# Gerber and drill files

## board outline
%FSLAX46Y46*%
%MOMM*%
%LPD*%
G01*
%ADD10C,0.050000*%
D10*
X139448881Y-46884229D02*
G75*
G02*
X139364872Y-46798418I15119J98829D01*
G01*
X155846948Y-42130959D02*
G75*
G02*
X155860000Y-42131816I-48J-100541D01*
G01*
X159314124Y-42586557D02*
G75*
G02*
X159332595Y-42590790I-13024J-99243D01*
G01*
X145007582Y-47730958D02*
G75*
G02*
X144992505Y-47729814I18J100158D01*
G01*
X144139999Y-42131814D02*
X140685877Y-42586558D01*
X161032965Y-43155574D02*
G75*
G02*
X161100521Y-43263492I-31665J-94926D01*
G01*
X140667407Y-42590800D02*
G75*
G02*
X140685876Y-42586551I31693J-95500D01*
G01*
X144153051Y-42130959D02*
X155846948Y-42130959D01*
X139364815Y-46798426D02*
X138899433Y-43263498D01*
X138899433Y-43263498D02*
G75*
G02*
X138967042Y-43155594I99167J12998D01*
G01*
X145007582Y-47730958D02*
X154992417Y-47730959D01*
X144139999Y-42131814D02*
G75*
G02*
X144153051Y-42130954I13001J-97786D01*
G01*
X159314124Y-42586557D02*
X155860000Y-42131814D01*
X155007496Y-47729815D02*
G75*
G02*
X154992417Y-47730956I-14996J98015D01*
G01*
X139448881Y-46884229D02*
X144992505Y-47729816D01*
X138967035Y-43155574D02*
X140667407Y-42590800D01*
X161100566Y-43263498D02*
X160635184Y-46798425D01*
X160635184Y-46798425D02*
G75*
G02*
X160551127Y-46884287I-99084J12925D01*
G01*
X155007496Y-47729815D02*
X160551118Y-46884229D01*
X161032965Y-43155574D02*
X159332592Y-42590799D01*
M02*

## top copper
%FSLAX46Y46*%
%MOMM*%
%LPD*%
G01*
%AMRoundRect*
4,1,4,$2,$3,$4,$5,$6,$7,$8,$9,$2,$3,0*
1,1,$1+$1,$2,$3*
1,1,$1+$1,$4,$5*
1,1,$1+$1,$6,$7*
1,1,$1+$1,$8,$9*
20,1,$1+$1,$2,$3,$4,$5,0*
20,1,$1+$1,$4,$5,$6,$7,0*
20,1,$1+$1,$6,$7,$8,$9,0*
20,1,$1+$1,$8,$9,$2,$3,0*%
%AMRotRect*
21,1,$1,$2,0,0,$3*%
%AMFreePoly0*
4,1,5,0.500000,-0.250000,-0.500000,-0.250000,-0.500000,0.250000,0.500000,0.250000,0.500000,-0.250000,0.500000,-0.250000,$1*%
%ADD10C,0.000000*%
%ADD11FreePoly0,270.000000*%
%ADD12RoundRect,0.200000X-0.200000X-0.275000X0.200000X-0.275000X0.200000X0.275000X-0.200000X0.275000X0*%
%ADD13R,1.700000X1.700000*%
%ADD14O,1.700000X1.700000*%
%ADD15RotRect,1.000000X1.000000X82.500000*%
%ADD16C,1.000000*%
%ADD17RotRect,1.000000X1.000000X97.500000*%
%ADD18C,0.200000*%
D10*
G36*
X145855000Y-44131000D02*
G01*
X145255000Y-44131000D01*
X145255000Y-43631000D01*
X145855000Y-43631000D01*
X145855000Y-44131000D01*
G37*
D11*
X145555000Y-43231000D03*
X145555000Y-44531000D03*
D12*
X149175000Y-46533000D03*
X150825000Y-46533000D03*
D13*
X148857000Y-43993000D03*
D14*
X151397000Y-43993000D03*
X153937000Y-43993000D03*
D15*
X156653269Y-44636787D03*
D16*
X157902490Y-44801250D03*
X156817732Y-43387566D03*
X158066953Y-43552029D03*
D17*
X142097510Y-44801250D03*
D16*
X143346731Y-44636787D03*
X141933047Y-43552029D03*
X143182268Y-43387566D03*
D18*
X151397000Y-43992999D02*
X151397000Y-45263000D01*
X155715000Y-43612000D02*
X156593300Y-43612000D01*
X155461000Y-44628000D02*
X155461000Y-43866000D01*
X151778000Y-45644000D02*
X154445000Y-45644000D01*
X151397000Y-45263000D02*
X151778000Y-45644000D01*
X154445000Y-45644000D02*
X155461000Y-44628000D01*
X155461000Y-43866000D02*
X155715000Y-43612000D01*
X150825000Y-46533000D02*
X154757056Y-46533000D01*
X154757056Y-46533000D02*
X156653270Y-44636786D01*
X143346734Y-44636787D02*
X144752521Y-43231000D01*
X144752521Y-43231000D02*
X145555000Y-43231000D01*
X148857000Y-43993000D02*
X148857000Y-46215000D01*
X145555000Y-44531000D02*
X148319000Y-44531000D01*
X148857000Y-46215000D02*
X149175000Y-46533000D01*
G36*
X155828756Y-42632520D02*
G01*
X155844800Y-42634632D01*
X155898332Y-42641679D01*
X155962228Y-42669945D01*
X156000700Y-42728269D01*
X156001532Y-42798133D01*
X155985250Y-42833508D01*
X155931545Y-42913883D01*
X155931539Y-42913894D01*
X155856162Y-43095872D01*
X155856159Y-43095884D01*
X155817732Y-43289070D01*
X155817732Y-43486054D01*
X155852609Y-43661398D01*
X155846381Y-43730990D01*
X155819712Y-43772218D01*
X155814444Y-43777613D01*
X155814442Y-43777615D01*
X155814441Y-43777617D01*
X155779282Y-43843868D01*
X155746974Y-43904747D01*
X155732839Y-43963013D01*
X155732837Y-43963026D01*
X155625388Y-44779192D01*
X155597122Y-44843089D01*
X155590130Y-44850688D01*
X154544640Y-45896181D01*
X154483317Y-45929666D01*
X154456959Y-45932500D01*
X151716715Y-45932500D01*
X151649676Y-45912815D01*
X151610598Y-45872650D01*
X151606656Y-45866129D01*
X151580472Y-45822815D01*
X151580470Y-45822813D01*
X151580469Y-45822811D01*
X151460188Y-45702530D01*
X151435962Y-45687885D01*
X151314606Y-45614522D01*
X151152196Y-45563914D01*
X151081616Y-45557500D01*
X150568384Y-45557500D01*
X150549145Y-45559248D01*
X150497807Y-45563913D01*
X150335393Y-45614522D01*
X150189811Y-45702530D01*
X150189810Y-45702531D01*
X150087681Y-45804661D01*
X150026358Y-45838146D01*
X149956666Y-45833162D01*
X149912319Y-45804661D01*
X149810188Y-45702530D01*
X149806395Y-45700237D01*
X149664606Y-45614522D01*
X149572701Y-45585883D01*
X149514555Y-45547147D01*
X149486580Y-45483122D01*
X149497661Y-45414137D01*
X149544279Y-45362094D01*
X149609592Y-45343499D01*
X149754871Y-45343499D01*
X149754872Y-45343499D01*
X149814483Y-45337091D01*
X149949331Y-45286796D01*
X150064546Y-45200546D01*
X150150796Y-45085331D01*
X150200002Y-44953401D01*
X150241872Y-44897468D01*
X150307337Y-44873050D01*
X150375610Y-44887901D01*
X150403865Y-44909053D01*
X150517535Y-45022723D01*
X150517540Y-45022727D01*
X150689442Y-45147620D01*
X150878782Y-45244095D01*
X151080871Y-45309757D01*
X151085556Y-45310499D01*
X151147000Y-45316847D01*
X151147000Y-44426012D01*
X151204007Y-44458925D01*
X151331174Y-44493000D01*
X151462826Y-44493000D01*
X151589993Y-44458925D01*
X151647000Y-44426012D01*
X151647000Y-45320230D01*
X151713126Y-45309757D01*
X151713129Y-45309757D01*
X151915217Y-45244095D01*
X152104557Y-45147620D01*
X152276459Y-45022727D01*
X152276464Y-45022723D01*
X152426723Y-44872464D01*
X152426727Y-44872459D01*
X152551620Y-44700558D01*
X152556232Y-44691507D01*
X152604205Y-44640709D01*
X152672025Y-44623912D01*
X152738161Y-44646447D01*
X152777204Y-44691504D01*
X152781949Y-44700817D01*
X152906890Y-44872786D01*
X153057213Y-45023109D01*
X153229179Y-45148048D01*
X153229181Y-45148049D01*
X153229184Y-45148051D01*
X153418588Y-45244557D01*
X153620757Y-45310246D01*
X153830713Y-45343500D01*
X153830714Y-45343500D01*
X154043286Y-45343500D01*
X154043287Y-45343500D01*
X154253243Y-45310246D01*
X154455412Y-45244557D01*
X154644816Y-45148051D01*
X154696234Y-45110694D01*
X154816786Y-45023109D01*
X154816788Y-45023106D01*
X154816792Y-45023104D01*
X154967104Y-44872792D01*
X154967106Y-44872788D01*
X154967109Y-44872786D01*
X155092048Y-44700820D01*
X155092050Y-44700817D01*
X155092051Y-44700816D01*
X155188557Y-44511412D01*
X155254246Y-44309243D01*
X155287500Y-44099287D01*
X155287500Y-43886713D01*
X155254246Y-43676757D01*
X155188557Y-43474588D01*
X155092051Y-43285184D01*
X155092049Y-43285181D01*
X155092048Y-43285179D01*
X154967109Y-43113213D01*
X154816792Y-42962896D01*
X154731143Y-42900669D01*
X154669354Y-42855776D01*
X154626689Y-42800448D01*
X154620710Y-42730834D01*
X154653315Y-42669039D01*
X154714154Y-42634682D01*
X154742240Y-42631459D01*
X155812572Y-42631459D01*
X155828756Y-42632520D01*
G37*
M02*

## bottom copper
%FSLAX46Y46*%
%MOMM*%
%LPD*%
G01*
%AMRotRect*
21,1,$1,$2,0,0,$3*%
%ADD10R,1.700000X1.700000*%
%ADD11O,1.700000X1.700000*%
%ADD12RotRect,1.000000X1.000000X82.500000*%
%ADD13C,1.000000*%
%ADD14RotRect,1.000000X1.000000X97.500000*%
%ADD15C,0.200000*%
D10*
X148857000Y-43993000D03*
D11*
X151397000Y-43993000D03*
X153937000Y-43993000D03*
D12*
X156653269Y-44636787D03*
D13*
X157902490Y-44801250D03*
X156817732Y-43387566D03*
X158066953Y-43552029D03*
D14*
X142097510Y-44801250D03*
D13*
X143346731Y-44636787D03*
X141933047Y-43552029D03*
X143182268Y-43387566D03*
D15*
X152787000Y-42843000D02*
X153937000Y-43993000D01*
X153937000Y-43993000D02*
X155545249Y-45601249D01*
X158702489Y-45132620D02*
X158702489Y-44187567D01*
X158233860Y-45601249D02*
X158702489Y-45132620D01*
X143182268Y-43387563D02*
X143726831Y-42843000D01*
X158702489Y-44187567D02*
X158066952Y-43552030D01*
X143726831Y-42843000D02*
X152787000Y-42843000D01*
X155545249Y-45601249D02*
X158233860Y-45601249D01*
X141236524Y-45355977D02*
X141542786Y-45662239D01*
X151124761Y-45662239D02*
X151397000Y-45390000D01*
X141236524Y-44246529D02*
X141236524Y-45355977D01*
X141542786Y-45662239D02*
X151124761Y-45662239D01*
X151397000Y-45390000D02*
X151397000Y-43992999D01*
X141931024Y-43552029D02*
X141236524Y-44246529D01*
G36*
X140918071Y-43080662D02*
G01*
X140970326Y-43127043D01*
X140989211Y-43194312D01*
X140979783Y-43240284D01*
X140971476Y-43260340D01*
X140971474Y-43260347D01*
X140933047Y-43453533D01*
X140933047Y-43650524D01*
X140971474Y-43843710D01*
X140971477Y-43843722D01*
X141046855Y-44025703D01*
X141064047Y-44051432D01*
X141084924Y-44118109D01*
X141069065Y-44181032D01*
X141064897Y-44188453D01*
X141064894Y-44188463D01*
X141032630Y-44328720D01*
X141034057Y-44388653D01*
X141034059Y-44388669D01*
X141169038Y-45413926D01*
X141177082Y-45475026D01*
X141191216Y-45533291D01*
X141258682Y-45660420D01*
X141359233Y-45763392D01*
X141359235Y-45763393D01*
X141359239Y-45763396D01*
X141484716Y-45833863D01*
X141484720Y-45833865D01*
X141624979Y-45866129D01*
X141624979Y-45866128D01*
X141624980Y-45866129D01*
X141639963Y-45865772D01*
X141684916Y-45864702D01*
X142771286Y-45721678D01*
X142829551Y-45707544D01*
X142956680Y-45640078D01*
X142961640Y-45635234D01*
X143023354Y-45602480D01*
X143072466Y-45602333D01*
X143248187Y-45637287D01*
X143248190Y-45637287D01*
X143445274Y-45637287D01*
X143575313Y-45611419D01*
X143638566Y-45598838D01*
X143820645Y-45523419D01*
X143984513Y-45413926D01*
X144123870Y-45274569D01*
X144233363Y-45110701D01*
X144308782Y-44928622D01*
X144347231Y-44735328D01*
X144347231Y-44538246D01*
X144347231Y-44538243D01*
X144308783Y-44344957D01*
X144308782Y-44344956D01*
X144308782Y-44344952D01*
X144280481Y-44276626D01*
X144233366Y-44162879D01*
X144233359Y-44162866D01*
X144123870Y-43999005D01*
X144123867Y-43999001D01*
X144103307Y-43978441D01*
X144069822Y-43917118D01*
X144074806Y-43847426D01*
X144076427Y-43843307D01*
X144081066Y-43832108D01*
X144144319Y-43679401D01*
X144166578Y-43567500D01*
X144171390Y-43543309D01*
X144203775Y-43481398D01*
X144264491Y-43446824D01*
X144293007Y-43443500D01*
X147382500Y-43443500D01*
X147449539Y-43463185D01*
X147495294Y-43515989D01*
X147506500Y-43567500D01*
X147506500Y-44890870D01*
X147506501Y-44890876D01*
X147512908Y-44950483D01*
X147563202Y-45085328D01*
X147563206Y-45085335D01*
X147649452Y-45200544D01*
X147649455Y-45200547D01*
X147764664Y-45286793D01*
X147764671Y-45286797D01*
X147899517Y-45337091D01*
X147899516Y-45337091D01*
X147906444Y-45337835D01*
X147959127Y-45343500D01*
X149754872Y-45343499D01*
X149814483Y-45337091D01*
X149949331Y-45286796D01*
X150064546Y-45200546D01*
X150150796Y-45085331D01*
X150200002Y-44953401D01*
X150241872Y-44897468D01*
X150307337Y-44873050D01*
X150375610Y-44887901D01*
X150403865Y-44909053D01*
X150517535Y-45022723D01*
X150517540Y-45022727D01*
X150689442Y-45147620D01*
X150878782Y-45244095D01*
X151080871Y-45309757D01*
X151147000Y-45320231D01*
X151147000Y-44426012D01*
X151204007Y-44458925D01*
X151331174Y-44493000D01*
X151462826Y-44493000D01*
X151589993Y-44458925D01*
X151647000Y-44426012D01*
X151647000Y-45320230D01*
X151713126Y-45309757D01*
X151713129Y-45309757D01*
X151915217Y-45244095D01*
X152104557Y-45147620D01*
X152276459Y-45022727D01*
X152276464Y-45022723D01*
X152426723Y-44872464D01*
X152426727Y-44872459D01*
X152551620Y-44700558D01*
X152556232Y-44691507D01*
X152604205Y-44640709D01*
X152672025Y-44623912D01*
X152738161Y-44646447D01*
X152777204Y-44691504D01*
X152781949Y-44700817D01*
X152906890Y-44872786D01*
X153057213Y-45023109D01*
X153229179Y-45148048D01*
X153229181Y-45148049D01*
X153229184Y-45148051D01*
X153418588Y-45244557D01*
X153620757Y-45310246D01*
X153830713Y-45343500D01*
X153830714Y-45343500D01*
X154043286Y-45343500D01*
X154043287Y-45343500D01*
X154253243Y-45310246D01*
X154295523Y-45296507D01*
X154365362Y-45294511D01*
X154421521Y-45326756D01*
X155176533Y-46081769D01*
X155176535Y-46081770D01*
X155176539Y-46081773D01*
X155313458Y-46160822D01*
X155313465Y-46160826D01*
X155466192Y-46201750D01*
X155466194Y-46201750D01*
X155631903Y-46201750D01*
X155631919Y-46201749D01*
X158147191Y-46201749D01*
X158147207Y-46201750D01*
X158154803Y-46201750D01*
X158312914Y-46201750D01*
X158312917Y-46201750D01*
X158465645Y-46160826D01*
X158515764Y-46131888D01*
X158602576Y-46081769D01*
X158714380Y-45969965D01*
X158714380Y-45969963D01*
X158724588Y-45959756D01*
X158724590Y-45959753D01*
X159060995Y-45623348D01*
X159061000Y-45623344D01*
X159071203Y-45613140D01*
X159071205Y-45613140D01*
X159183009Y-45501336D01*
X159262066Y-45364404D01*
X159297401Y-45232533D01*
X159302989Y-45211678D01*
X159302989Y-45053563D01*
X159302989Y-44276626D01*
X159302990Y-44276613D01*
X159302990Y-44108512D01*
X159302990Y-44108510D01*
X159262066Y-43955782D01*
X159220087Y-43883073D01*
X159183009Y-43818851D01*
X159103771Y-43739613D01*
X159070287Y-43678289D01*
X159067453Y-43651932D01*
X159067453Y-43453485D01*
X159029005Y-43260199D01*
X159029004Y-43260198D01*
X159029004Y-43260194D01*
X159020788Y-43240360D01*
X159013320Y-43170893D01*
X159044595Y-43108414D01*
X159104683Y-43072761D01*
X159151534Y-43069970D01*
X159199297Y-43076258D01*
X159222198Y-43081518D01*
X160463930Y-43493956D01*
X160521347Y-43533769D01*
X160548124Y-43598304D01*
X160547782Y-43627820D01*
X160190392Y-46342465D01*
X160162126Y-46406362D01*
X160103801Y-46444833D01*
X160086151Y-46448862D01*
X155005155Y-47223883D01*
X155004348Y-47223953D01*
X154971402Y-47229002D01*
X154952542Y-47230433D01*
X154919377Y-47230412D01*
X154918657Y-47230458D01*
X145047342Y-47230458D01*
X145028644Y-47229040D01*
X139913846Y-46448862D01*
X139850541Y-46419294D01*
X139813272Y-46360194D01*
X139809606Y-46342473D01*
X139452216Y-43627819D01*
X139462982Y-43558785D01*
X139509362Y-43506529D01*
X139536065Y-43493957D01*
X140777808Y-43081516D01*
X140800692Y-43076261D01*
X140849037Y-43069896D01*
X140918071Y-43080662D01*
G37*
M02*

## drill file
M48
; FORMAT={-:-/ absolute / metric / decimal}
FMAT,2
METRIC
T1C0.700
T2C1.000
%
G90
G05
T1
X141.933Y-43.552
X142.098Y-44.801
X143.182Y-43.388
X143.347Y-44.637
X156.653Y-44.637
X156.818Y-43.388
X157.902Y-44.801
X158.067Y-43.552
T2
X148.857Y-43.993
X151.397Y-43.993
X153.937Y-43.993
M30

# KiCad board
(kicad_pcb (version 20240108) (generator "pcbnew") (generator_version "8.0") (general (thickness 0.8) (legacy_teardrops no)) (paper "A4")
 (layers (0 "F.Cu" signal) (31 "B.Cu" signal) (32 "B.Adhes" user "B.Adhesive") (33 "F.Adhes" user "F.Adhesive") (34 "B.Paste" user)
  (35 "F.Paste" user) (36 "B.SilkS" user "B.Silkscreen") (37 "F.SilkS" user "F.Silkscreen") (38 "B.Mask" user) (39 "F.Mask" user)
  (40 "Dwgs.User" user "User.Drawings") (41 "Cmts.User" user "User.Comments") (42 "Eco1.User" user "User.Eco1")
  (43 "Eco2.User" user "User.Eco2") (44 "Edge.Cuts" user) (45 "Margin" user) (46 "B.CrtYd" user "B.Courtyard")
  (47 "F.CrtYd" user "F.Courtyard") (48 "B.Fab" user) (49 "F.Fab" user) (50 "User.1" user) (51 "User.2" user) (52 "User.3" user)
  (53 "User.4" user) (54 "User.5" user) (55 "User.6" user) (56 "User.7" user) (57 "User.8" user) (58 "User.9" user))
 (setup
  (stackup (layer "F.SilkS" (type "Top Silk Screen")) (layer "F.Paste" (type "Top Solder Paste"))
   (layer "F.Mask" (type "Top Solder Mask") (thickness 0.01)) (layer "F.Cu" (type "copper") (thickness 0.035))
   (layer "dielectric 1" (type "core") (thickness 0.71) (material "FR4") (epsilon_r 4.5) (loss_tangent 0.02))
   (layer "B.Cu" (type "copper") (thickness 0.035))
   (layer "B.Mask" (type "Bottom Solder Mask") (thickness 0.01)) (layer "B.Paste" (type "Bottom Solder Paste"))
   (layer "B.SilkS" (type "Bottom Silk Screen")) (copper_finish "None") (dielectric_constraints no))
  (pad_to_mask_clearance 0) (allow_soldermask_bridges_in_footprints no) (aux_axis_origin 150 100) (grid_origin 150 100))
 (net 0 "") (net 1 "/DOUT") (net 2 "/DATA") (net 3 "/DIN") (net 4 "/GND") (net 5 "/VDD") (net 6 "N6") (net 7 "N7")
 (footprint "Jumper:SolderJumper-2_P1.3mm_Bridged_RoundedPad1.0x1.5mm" (layer "F.Cu") (at 145.555 43.881 -90)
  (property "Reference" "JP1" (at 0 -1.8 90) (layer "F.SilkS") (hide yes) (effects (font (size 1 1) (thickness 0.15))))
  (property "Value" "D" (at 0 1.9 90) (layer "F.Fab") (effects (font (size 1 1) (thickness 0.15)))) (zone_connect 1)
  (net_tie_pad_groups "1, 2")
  (fp_poly (pts (xy 0.25 -0.3) (xy -0.25 -0.3) (xy -0.25 0.3) (xy 0.25 0.3)) (stroke (width 0) (type solid)) (fill solid) (layer "F.Cu"))
  (pad "1" smd custom (at -0.65 0 270) (size 1 0.5) (layers "F.Cu" "F.Mask") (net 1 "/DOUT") (zone_connect 2) (thermal_bridge_angle 45)
   (options (clearance outline) (anchor rect)) (primitives))
  (pad "2" smd custom (at 0.65 0 270) (size 1 0.5) (layers "F.Cu" "F.Mask") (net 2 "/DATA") (zone_connect 2) (thermal_bridge_angle 45)
   (options (clearance outline) (anchor rect)) (primitives)))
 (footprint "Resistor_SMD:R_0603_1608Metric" (layer "F.Cu") (at 150 46.533)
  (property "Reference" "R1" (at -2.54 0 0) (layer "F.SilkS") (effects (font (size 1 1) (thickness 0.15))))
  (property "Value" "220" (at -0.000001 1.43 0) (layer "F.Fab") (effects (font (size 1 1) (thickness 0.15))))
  (pad "1" smd roundrect (at -0.825 0) (size 0.8 0.95) (layers "F.Cu" "F.Paste" "F.Mask") (roundrect_rratio 0.25) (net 2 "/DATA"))
  (pad "2" smd roundrect (at 0.825 0) (size 0.8 0.95) (layers "F.Cu" "F.Paste" "F.Mask") (roundrect_rratio 0.25) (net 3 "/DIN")))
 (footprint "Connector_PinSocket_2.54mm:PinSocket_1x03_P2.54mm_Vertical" (layer "F.Cu") (at 148.857 43.993 90)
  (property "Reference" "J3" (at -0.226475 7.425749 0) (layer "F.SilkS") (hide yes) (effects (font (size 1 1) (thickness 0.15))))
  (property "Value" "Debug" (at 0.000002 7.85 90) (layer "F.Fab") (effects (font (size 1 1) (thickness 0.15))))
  (pad "1" thru_hole rect (at 0 0 90) (size 1.7 1.7) (drill 1) (layers "*.Cu" "*.Mask") (remove_unused_layers no) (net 2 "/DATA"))
  (pad "2" thru_hole oval (at 0 2.54 90) (size 1.7 1.7) (drill 1) (layers "*.Cu" "*.Mask") (remove_unused_layers no) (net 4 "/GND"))
  (pad "3" thru_hole oval (at 0 5.08 90) (size 1.7 1.7) (drill 1) (layers "*.Cu" "*.Mask") (remove_unused_layers no) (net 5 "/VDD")))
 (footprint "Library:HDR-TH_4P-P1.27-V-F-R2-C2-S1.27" (layer "B.Cu") (at 157.360111 44.094408 82.5)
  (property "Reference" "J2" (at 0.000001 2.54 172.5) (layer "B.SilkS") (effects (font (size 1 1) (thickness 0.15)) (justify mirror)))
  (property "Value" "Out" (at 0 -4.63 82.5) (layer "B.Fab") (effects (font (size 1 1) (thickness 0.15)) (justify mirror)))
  (pad "1" thru_hole rect (at -0.63 -0.63 82.5) (size 1 1) (drill 0.700024) (layers "*.Cu" "*.Mask") (remove_unused_layers no)
   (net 3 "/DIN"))
  (pad "2" thru_hole circle (at -0.63 0.63 82.5) (size 1 1) (drill 0.700024) (layers "*.Cu" "*.Mask") (remove_unused_layers no) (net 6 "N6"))
  (pad "3" thru_hole circle (at 0.63 -0.63 82.5) (size 1 1) (drill 0.700024) (layers "*.Cu" "*.Mask") (remove_unused_layers no)
   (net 4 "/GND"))
  (pad "4" thru_hole circle (at 0.63 0.63 82.5) (size 1 1) (drill 0.700024) (layers "*.Cu" "*.Mask") (remove_unused_layers no)
   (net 5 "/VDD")))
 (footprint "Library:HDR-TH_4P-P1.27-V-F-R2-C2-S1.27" (layer "B.Cu") (at 142.639889 44.094408 97.5)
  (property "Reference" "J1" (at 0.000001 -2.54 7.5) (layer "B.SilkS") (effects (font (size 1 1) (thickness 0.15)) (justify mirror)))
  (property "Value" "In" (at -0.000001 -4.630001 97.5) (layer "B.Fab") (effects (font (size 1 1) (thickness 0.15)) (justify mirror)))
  (pad "1" thru_hole rect (at -0.63 -0.63 97.5) (size 1 1) (drill 0.700024) (layers "*.Cu" "*.Mask") (remove_unused_layers no) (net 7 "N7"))
  (pad "2" thru_hole circle (at -0.63 0.63 97.5) (size 1 1) (drill 0.700024) (layers "*.Cu" "*.Mask") (remove_unused_layers no)
   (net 1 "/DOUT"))
  (pad "3" thru_hole circle (at 0.63 -0.63 97.5) (size 1 1) (drill 0.700024) (layers "*.Cu" "*.Mask") (remove_unused_layers no)
   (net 4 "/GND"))
  (pad "4" thru_hole circle (at 0.63 0.63 97.5) (size 1 1) (drill 0.700024) (layers "*.Cu" "*.Mask") (remove_unused_layers no)
   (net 5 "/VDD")))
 (gr_arc (start 139.448881 46.884229) (mid 139.392529 46.855356) (end 139.364815 46.798426) (stroke (width 0.05) (type default))
  (layer "Edge.Cuts"))
 (gr_arc (start 155.846948 42.130959) (mid 155.853488 42.131174) (end 155.86 42.131814) (stroke (width 0.05) (type default))
  (layer "Edge.Cuts"))
 (gr_arc (start 159.314124 42.586557) (mid 159.323459 42.58824) (end 159.332592 42.590799) (stroke (width 0.05) (type default))
  (layer "Edge.Cuts"))
 (gr_arc (start 145.007582 47.730958) (mid 145.000022 47.730672) (end 144.992505 47.729816) (stroke (width 0.05) (type default))
  (layer "Edge.Cuts"))
 (gr_line (start 144.139999 42.131814) (end 140.685877 42.586558) (stroke (width 0.05) (type default)) (layer "Edge.Cuts"))
 (gr_arc (start 161.032965 43.155574) (mid 161.086144 43.197387) (end 161.100566 43.263498) (stroke (width 0.05) (type default))
  (layer "Edge.Cuts"))
 (gr_arc (start 140.667407 42.5908) (mid 140.676542 42.588243) (end 140.685877 42.586558) (stroke (width 0.05) (type default))
  (layer "Edge.Cuts"))
 (gr_line (start 144.153051 42.130959) (end 155.846948 42.130959) (stroke (width 0.05) (type default)) (layer "Edge.Cuts"))
 (gr_line (start 139.364815 46.798426) (end 138.899433 43.263498) (stroke (width 0.05) (type default)) (layer "Edge.Cuts"))
 (gr_arc (start 138.899433 43.263498) (mid 138.913836 43.197386) (end 138.967035 43.155574) (stroke (width 0.05) (type default))
  (layer "Edge.Cuts"))
 (gr_line (start 145.007582 47.730958) (end 154.992417 47.730959) (stroke (width 0.05) (type default)) (layer "Edge.Cuts"))
 (gr_arc (start 144.139999 42.131814) (mid 144.146511 42.13117) (end 144.153051 42.130959) (stroke (width 0.05) (type default))
  (layer "Edge.Cuts"))
 (gr_line (start 159.314124 42.586557) (end 155.86 42.131814) (stroke (width 0.05) (type default)) (layer "Edge.Cuts"))
 (gr_arc (start 155.007496 47.729815) (mid 154.999978 47.730675) (end 154.992417 47.730959) (stroke (width 0.05) (type default))
  (layer "Edge.Cuts"))
 (gr_line (start 139.448881 46.884229) (end 144.992505 47.729816) (stroke (width 0.05) (type default)) (layer "Edge.Cuts"))
 (gr_line (start 138.967035 43.155574) (end 140.667407 42.5908) (stroke (width 0.05) (type default)) (layer "Edge.Cuts"))
 (gr_line (start 161.100566 43.263498) (end 160.635184 46.798425) (stroke (width 0.05) (type default)) (layer "Edge.Cuts"))
 (gr_arc (start 160.635184 46.798425) (mid 160.607482 46.855376) (end 160.551118 46.884229) (stroke (width 0.05) (type default))
  (layer "Edge.Cuts"))
 (gr_line (start 155.007496 47.729815) (end 160.551118 46.884229) (stroke (width 0.05) (type default)) (layer "Edge.Cuts"))
 (gr_line (start 161.032965 43.155574) (end 159.332592 42.590799) (stroke (width 0.05) (type default)) (layer "Edge.Cuts"))
 (segment (start 152.787 42.843) (end 153.937 43.993) (width 0.2) (layer "B.Cu") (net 5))
 (segment (start 153.937 43.993) (end 155.545249 45.601249) (width 0.2) (layer "B.Cu") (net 5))
 (segment (start 158.702489 45.13262) (end 158.702489 44.187567) (width 0.2) (layer "B.Cu") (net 5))
 (segment (start 158.23386 45.601249) (end 158.702489 45.13262) (width 0.2) (layer "B.Cu") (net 5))
 (segment (start 143.182268 43.387563) (end 143.726831 42.843) (width 0.2) (layer "B.Cu") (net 5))
 (segment (start 158.702489 44.187567) (end 158.066952 43.55203) (width 0.2) (layer "B.Cu") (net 5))
 (segment (start 143.726831 42.843) (end 152.787 42.843) (width 0.2) (layer "B.Cu") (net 5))
 (segment (start 155.545249 45.601249) (end 158.23386 45.601249) (width 0.2) (layer "B.Cu") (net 5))
 (segment (start 151.397 43.992999) (end 151.397 45.263) (width 0.2) (layer "F.Cu") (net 4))
 (segment (start 155.715 43.612) (end 156.5933 43.612) (width 0.2) (layer "F.Cu") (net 4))
 (segment (start 155.461 44.628) (end 155.461 43.866) (width 0.2) (layer "F.Cu") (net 4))
 (segment (start 151.778 45.644) (end 154.445 45.644) (width 0.2) (layer "F.Cu") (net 4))
 (segment (start 151.397 45.263) (end 151.778 45.644) (width 0.2) (layer "F.Cu") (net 4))
 (segment (start 154.445 45.644) (end 155.461 44.628) (width 0.2) (layer "F.Cu") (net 4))
 (segment (start 155.461 43.866) (end 155.715 43.612) (width 0.2) (layer "F.Cu") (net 4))
 (segment (start 141.236524 45.355977) (end 141.542786 45.662239) (width 0.2) (layer "B.Cu") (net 4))
 (segment (start 151.124761 45.662239) (end 151.397 45.39) (width 0.2) (layer "B.Cu") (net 4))
 (segment (start 141.236524 44.246529) (end 141.236524 45.355977) (width 0.2) (layer "B.Cu") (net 4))
 (segment (start 141.542786 45.662239) (end 151.124761 45.662239) (width 0.2) (layer "B.Cu") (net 4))
 (segment (start 151.397 45.39) (end 151.397 43.992999) (width 0.2) (layer "B.Cu") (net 4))
 (segment (start 141.931024 43.552029) (end 141.236524 44.246529) (width 0.2) (layer "B.Cu") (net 4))
 (segment (start 150.825 46.533) (end 154.757056 46.533) (width 0.2) (layer "F.Cu") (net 3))
 (segment (start 154.757056 46.533) (end 156.65327 44.636786) (width 0.2) (layer "F.Cu") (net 3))
 (segment (start 143.346734 44.636787) (end 144.752521 43.231) (width 0.2) (layer "F.Cu") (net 1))
 (segment (start 144.752521 43.231) (end 145.555 43.231) (width 0.2) (layer "F.Cu") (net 1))
 (segment (start 148.857 43.993) (end 148.857 46.215) (width 0.2) (layer "F.Cu") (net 2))
 (segment (start 145.555 44.531) (end 148.319 44.531) (width 0.2) (layer "F.Cu") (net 2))
 (segment (start 148.857 46.215) (end 149.175 46.533) (width 0.2) (layer "F.Cu") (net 2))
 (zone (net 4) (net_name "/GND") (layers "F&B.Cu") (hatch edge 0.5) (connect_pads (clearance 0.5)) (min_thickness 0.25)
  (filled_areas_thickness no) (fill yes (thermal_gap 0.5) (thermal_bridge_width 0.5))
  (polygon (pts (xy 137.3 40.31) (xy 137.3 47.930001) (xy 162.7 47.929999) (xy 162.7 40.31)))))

